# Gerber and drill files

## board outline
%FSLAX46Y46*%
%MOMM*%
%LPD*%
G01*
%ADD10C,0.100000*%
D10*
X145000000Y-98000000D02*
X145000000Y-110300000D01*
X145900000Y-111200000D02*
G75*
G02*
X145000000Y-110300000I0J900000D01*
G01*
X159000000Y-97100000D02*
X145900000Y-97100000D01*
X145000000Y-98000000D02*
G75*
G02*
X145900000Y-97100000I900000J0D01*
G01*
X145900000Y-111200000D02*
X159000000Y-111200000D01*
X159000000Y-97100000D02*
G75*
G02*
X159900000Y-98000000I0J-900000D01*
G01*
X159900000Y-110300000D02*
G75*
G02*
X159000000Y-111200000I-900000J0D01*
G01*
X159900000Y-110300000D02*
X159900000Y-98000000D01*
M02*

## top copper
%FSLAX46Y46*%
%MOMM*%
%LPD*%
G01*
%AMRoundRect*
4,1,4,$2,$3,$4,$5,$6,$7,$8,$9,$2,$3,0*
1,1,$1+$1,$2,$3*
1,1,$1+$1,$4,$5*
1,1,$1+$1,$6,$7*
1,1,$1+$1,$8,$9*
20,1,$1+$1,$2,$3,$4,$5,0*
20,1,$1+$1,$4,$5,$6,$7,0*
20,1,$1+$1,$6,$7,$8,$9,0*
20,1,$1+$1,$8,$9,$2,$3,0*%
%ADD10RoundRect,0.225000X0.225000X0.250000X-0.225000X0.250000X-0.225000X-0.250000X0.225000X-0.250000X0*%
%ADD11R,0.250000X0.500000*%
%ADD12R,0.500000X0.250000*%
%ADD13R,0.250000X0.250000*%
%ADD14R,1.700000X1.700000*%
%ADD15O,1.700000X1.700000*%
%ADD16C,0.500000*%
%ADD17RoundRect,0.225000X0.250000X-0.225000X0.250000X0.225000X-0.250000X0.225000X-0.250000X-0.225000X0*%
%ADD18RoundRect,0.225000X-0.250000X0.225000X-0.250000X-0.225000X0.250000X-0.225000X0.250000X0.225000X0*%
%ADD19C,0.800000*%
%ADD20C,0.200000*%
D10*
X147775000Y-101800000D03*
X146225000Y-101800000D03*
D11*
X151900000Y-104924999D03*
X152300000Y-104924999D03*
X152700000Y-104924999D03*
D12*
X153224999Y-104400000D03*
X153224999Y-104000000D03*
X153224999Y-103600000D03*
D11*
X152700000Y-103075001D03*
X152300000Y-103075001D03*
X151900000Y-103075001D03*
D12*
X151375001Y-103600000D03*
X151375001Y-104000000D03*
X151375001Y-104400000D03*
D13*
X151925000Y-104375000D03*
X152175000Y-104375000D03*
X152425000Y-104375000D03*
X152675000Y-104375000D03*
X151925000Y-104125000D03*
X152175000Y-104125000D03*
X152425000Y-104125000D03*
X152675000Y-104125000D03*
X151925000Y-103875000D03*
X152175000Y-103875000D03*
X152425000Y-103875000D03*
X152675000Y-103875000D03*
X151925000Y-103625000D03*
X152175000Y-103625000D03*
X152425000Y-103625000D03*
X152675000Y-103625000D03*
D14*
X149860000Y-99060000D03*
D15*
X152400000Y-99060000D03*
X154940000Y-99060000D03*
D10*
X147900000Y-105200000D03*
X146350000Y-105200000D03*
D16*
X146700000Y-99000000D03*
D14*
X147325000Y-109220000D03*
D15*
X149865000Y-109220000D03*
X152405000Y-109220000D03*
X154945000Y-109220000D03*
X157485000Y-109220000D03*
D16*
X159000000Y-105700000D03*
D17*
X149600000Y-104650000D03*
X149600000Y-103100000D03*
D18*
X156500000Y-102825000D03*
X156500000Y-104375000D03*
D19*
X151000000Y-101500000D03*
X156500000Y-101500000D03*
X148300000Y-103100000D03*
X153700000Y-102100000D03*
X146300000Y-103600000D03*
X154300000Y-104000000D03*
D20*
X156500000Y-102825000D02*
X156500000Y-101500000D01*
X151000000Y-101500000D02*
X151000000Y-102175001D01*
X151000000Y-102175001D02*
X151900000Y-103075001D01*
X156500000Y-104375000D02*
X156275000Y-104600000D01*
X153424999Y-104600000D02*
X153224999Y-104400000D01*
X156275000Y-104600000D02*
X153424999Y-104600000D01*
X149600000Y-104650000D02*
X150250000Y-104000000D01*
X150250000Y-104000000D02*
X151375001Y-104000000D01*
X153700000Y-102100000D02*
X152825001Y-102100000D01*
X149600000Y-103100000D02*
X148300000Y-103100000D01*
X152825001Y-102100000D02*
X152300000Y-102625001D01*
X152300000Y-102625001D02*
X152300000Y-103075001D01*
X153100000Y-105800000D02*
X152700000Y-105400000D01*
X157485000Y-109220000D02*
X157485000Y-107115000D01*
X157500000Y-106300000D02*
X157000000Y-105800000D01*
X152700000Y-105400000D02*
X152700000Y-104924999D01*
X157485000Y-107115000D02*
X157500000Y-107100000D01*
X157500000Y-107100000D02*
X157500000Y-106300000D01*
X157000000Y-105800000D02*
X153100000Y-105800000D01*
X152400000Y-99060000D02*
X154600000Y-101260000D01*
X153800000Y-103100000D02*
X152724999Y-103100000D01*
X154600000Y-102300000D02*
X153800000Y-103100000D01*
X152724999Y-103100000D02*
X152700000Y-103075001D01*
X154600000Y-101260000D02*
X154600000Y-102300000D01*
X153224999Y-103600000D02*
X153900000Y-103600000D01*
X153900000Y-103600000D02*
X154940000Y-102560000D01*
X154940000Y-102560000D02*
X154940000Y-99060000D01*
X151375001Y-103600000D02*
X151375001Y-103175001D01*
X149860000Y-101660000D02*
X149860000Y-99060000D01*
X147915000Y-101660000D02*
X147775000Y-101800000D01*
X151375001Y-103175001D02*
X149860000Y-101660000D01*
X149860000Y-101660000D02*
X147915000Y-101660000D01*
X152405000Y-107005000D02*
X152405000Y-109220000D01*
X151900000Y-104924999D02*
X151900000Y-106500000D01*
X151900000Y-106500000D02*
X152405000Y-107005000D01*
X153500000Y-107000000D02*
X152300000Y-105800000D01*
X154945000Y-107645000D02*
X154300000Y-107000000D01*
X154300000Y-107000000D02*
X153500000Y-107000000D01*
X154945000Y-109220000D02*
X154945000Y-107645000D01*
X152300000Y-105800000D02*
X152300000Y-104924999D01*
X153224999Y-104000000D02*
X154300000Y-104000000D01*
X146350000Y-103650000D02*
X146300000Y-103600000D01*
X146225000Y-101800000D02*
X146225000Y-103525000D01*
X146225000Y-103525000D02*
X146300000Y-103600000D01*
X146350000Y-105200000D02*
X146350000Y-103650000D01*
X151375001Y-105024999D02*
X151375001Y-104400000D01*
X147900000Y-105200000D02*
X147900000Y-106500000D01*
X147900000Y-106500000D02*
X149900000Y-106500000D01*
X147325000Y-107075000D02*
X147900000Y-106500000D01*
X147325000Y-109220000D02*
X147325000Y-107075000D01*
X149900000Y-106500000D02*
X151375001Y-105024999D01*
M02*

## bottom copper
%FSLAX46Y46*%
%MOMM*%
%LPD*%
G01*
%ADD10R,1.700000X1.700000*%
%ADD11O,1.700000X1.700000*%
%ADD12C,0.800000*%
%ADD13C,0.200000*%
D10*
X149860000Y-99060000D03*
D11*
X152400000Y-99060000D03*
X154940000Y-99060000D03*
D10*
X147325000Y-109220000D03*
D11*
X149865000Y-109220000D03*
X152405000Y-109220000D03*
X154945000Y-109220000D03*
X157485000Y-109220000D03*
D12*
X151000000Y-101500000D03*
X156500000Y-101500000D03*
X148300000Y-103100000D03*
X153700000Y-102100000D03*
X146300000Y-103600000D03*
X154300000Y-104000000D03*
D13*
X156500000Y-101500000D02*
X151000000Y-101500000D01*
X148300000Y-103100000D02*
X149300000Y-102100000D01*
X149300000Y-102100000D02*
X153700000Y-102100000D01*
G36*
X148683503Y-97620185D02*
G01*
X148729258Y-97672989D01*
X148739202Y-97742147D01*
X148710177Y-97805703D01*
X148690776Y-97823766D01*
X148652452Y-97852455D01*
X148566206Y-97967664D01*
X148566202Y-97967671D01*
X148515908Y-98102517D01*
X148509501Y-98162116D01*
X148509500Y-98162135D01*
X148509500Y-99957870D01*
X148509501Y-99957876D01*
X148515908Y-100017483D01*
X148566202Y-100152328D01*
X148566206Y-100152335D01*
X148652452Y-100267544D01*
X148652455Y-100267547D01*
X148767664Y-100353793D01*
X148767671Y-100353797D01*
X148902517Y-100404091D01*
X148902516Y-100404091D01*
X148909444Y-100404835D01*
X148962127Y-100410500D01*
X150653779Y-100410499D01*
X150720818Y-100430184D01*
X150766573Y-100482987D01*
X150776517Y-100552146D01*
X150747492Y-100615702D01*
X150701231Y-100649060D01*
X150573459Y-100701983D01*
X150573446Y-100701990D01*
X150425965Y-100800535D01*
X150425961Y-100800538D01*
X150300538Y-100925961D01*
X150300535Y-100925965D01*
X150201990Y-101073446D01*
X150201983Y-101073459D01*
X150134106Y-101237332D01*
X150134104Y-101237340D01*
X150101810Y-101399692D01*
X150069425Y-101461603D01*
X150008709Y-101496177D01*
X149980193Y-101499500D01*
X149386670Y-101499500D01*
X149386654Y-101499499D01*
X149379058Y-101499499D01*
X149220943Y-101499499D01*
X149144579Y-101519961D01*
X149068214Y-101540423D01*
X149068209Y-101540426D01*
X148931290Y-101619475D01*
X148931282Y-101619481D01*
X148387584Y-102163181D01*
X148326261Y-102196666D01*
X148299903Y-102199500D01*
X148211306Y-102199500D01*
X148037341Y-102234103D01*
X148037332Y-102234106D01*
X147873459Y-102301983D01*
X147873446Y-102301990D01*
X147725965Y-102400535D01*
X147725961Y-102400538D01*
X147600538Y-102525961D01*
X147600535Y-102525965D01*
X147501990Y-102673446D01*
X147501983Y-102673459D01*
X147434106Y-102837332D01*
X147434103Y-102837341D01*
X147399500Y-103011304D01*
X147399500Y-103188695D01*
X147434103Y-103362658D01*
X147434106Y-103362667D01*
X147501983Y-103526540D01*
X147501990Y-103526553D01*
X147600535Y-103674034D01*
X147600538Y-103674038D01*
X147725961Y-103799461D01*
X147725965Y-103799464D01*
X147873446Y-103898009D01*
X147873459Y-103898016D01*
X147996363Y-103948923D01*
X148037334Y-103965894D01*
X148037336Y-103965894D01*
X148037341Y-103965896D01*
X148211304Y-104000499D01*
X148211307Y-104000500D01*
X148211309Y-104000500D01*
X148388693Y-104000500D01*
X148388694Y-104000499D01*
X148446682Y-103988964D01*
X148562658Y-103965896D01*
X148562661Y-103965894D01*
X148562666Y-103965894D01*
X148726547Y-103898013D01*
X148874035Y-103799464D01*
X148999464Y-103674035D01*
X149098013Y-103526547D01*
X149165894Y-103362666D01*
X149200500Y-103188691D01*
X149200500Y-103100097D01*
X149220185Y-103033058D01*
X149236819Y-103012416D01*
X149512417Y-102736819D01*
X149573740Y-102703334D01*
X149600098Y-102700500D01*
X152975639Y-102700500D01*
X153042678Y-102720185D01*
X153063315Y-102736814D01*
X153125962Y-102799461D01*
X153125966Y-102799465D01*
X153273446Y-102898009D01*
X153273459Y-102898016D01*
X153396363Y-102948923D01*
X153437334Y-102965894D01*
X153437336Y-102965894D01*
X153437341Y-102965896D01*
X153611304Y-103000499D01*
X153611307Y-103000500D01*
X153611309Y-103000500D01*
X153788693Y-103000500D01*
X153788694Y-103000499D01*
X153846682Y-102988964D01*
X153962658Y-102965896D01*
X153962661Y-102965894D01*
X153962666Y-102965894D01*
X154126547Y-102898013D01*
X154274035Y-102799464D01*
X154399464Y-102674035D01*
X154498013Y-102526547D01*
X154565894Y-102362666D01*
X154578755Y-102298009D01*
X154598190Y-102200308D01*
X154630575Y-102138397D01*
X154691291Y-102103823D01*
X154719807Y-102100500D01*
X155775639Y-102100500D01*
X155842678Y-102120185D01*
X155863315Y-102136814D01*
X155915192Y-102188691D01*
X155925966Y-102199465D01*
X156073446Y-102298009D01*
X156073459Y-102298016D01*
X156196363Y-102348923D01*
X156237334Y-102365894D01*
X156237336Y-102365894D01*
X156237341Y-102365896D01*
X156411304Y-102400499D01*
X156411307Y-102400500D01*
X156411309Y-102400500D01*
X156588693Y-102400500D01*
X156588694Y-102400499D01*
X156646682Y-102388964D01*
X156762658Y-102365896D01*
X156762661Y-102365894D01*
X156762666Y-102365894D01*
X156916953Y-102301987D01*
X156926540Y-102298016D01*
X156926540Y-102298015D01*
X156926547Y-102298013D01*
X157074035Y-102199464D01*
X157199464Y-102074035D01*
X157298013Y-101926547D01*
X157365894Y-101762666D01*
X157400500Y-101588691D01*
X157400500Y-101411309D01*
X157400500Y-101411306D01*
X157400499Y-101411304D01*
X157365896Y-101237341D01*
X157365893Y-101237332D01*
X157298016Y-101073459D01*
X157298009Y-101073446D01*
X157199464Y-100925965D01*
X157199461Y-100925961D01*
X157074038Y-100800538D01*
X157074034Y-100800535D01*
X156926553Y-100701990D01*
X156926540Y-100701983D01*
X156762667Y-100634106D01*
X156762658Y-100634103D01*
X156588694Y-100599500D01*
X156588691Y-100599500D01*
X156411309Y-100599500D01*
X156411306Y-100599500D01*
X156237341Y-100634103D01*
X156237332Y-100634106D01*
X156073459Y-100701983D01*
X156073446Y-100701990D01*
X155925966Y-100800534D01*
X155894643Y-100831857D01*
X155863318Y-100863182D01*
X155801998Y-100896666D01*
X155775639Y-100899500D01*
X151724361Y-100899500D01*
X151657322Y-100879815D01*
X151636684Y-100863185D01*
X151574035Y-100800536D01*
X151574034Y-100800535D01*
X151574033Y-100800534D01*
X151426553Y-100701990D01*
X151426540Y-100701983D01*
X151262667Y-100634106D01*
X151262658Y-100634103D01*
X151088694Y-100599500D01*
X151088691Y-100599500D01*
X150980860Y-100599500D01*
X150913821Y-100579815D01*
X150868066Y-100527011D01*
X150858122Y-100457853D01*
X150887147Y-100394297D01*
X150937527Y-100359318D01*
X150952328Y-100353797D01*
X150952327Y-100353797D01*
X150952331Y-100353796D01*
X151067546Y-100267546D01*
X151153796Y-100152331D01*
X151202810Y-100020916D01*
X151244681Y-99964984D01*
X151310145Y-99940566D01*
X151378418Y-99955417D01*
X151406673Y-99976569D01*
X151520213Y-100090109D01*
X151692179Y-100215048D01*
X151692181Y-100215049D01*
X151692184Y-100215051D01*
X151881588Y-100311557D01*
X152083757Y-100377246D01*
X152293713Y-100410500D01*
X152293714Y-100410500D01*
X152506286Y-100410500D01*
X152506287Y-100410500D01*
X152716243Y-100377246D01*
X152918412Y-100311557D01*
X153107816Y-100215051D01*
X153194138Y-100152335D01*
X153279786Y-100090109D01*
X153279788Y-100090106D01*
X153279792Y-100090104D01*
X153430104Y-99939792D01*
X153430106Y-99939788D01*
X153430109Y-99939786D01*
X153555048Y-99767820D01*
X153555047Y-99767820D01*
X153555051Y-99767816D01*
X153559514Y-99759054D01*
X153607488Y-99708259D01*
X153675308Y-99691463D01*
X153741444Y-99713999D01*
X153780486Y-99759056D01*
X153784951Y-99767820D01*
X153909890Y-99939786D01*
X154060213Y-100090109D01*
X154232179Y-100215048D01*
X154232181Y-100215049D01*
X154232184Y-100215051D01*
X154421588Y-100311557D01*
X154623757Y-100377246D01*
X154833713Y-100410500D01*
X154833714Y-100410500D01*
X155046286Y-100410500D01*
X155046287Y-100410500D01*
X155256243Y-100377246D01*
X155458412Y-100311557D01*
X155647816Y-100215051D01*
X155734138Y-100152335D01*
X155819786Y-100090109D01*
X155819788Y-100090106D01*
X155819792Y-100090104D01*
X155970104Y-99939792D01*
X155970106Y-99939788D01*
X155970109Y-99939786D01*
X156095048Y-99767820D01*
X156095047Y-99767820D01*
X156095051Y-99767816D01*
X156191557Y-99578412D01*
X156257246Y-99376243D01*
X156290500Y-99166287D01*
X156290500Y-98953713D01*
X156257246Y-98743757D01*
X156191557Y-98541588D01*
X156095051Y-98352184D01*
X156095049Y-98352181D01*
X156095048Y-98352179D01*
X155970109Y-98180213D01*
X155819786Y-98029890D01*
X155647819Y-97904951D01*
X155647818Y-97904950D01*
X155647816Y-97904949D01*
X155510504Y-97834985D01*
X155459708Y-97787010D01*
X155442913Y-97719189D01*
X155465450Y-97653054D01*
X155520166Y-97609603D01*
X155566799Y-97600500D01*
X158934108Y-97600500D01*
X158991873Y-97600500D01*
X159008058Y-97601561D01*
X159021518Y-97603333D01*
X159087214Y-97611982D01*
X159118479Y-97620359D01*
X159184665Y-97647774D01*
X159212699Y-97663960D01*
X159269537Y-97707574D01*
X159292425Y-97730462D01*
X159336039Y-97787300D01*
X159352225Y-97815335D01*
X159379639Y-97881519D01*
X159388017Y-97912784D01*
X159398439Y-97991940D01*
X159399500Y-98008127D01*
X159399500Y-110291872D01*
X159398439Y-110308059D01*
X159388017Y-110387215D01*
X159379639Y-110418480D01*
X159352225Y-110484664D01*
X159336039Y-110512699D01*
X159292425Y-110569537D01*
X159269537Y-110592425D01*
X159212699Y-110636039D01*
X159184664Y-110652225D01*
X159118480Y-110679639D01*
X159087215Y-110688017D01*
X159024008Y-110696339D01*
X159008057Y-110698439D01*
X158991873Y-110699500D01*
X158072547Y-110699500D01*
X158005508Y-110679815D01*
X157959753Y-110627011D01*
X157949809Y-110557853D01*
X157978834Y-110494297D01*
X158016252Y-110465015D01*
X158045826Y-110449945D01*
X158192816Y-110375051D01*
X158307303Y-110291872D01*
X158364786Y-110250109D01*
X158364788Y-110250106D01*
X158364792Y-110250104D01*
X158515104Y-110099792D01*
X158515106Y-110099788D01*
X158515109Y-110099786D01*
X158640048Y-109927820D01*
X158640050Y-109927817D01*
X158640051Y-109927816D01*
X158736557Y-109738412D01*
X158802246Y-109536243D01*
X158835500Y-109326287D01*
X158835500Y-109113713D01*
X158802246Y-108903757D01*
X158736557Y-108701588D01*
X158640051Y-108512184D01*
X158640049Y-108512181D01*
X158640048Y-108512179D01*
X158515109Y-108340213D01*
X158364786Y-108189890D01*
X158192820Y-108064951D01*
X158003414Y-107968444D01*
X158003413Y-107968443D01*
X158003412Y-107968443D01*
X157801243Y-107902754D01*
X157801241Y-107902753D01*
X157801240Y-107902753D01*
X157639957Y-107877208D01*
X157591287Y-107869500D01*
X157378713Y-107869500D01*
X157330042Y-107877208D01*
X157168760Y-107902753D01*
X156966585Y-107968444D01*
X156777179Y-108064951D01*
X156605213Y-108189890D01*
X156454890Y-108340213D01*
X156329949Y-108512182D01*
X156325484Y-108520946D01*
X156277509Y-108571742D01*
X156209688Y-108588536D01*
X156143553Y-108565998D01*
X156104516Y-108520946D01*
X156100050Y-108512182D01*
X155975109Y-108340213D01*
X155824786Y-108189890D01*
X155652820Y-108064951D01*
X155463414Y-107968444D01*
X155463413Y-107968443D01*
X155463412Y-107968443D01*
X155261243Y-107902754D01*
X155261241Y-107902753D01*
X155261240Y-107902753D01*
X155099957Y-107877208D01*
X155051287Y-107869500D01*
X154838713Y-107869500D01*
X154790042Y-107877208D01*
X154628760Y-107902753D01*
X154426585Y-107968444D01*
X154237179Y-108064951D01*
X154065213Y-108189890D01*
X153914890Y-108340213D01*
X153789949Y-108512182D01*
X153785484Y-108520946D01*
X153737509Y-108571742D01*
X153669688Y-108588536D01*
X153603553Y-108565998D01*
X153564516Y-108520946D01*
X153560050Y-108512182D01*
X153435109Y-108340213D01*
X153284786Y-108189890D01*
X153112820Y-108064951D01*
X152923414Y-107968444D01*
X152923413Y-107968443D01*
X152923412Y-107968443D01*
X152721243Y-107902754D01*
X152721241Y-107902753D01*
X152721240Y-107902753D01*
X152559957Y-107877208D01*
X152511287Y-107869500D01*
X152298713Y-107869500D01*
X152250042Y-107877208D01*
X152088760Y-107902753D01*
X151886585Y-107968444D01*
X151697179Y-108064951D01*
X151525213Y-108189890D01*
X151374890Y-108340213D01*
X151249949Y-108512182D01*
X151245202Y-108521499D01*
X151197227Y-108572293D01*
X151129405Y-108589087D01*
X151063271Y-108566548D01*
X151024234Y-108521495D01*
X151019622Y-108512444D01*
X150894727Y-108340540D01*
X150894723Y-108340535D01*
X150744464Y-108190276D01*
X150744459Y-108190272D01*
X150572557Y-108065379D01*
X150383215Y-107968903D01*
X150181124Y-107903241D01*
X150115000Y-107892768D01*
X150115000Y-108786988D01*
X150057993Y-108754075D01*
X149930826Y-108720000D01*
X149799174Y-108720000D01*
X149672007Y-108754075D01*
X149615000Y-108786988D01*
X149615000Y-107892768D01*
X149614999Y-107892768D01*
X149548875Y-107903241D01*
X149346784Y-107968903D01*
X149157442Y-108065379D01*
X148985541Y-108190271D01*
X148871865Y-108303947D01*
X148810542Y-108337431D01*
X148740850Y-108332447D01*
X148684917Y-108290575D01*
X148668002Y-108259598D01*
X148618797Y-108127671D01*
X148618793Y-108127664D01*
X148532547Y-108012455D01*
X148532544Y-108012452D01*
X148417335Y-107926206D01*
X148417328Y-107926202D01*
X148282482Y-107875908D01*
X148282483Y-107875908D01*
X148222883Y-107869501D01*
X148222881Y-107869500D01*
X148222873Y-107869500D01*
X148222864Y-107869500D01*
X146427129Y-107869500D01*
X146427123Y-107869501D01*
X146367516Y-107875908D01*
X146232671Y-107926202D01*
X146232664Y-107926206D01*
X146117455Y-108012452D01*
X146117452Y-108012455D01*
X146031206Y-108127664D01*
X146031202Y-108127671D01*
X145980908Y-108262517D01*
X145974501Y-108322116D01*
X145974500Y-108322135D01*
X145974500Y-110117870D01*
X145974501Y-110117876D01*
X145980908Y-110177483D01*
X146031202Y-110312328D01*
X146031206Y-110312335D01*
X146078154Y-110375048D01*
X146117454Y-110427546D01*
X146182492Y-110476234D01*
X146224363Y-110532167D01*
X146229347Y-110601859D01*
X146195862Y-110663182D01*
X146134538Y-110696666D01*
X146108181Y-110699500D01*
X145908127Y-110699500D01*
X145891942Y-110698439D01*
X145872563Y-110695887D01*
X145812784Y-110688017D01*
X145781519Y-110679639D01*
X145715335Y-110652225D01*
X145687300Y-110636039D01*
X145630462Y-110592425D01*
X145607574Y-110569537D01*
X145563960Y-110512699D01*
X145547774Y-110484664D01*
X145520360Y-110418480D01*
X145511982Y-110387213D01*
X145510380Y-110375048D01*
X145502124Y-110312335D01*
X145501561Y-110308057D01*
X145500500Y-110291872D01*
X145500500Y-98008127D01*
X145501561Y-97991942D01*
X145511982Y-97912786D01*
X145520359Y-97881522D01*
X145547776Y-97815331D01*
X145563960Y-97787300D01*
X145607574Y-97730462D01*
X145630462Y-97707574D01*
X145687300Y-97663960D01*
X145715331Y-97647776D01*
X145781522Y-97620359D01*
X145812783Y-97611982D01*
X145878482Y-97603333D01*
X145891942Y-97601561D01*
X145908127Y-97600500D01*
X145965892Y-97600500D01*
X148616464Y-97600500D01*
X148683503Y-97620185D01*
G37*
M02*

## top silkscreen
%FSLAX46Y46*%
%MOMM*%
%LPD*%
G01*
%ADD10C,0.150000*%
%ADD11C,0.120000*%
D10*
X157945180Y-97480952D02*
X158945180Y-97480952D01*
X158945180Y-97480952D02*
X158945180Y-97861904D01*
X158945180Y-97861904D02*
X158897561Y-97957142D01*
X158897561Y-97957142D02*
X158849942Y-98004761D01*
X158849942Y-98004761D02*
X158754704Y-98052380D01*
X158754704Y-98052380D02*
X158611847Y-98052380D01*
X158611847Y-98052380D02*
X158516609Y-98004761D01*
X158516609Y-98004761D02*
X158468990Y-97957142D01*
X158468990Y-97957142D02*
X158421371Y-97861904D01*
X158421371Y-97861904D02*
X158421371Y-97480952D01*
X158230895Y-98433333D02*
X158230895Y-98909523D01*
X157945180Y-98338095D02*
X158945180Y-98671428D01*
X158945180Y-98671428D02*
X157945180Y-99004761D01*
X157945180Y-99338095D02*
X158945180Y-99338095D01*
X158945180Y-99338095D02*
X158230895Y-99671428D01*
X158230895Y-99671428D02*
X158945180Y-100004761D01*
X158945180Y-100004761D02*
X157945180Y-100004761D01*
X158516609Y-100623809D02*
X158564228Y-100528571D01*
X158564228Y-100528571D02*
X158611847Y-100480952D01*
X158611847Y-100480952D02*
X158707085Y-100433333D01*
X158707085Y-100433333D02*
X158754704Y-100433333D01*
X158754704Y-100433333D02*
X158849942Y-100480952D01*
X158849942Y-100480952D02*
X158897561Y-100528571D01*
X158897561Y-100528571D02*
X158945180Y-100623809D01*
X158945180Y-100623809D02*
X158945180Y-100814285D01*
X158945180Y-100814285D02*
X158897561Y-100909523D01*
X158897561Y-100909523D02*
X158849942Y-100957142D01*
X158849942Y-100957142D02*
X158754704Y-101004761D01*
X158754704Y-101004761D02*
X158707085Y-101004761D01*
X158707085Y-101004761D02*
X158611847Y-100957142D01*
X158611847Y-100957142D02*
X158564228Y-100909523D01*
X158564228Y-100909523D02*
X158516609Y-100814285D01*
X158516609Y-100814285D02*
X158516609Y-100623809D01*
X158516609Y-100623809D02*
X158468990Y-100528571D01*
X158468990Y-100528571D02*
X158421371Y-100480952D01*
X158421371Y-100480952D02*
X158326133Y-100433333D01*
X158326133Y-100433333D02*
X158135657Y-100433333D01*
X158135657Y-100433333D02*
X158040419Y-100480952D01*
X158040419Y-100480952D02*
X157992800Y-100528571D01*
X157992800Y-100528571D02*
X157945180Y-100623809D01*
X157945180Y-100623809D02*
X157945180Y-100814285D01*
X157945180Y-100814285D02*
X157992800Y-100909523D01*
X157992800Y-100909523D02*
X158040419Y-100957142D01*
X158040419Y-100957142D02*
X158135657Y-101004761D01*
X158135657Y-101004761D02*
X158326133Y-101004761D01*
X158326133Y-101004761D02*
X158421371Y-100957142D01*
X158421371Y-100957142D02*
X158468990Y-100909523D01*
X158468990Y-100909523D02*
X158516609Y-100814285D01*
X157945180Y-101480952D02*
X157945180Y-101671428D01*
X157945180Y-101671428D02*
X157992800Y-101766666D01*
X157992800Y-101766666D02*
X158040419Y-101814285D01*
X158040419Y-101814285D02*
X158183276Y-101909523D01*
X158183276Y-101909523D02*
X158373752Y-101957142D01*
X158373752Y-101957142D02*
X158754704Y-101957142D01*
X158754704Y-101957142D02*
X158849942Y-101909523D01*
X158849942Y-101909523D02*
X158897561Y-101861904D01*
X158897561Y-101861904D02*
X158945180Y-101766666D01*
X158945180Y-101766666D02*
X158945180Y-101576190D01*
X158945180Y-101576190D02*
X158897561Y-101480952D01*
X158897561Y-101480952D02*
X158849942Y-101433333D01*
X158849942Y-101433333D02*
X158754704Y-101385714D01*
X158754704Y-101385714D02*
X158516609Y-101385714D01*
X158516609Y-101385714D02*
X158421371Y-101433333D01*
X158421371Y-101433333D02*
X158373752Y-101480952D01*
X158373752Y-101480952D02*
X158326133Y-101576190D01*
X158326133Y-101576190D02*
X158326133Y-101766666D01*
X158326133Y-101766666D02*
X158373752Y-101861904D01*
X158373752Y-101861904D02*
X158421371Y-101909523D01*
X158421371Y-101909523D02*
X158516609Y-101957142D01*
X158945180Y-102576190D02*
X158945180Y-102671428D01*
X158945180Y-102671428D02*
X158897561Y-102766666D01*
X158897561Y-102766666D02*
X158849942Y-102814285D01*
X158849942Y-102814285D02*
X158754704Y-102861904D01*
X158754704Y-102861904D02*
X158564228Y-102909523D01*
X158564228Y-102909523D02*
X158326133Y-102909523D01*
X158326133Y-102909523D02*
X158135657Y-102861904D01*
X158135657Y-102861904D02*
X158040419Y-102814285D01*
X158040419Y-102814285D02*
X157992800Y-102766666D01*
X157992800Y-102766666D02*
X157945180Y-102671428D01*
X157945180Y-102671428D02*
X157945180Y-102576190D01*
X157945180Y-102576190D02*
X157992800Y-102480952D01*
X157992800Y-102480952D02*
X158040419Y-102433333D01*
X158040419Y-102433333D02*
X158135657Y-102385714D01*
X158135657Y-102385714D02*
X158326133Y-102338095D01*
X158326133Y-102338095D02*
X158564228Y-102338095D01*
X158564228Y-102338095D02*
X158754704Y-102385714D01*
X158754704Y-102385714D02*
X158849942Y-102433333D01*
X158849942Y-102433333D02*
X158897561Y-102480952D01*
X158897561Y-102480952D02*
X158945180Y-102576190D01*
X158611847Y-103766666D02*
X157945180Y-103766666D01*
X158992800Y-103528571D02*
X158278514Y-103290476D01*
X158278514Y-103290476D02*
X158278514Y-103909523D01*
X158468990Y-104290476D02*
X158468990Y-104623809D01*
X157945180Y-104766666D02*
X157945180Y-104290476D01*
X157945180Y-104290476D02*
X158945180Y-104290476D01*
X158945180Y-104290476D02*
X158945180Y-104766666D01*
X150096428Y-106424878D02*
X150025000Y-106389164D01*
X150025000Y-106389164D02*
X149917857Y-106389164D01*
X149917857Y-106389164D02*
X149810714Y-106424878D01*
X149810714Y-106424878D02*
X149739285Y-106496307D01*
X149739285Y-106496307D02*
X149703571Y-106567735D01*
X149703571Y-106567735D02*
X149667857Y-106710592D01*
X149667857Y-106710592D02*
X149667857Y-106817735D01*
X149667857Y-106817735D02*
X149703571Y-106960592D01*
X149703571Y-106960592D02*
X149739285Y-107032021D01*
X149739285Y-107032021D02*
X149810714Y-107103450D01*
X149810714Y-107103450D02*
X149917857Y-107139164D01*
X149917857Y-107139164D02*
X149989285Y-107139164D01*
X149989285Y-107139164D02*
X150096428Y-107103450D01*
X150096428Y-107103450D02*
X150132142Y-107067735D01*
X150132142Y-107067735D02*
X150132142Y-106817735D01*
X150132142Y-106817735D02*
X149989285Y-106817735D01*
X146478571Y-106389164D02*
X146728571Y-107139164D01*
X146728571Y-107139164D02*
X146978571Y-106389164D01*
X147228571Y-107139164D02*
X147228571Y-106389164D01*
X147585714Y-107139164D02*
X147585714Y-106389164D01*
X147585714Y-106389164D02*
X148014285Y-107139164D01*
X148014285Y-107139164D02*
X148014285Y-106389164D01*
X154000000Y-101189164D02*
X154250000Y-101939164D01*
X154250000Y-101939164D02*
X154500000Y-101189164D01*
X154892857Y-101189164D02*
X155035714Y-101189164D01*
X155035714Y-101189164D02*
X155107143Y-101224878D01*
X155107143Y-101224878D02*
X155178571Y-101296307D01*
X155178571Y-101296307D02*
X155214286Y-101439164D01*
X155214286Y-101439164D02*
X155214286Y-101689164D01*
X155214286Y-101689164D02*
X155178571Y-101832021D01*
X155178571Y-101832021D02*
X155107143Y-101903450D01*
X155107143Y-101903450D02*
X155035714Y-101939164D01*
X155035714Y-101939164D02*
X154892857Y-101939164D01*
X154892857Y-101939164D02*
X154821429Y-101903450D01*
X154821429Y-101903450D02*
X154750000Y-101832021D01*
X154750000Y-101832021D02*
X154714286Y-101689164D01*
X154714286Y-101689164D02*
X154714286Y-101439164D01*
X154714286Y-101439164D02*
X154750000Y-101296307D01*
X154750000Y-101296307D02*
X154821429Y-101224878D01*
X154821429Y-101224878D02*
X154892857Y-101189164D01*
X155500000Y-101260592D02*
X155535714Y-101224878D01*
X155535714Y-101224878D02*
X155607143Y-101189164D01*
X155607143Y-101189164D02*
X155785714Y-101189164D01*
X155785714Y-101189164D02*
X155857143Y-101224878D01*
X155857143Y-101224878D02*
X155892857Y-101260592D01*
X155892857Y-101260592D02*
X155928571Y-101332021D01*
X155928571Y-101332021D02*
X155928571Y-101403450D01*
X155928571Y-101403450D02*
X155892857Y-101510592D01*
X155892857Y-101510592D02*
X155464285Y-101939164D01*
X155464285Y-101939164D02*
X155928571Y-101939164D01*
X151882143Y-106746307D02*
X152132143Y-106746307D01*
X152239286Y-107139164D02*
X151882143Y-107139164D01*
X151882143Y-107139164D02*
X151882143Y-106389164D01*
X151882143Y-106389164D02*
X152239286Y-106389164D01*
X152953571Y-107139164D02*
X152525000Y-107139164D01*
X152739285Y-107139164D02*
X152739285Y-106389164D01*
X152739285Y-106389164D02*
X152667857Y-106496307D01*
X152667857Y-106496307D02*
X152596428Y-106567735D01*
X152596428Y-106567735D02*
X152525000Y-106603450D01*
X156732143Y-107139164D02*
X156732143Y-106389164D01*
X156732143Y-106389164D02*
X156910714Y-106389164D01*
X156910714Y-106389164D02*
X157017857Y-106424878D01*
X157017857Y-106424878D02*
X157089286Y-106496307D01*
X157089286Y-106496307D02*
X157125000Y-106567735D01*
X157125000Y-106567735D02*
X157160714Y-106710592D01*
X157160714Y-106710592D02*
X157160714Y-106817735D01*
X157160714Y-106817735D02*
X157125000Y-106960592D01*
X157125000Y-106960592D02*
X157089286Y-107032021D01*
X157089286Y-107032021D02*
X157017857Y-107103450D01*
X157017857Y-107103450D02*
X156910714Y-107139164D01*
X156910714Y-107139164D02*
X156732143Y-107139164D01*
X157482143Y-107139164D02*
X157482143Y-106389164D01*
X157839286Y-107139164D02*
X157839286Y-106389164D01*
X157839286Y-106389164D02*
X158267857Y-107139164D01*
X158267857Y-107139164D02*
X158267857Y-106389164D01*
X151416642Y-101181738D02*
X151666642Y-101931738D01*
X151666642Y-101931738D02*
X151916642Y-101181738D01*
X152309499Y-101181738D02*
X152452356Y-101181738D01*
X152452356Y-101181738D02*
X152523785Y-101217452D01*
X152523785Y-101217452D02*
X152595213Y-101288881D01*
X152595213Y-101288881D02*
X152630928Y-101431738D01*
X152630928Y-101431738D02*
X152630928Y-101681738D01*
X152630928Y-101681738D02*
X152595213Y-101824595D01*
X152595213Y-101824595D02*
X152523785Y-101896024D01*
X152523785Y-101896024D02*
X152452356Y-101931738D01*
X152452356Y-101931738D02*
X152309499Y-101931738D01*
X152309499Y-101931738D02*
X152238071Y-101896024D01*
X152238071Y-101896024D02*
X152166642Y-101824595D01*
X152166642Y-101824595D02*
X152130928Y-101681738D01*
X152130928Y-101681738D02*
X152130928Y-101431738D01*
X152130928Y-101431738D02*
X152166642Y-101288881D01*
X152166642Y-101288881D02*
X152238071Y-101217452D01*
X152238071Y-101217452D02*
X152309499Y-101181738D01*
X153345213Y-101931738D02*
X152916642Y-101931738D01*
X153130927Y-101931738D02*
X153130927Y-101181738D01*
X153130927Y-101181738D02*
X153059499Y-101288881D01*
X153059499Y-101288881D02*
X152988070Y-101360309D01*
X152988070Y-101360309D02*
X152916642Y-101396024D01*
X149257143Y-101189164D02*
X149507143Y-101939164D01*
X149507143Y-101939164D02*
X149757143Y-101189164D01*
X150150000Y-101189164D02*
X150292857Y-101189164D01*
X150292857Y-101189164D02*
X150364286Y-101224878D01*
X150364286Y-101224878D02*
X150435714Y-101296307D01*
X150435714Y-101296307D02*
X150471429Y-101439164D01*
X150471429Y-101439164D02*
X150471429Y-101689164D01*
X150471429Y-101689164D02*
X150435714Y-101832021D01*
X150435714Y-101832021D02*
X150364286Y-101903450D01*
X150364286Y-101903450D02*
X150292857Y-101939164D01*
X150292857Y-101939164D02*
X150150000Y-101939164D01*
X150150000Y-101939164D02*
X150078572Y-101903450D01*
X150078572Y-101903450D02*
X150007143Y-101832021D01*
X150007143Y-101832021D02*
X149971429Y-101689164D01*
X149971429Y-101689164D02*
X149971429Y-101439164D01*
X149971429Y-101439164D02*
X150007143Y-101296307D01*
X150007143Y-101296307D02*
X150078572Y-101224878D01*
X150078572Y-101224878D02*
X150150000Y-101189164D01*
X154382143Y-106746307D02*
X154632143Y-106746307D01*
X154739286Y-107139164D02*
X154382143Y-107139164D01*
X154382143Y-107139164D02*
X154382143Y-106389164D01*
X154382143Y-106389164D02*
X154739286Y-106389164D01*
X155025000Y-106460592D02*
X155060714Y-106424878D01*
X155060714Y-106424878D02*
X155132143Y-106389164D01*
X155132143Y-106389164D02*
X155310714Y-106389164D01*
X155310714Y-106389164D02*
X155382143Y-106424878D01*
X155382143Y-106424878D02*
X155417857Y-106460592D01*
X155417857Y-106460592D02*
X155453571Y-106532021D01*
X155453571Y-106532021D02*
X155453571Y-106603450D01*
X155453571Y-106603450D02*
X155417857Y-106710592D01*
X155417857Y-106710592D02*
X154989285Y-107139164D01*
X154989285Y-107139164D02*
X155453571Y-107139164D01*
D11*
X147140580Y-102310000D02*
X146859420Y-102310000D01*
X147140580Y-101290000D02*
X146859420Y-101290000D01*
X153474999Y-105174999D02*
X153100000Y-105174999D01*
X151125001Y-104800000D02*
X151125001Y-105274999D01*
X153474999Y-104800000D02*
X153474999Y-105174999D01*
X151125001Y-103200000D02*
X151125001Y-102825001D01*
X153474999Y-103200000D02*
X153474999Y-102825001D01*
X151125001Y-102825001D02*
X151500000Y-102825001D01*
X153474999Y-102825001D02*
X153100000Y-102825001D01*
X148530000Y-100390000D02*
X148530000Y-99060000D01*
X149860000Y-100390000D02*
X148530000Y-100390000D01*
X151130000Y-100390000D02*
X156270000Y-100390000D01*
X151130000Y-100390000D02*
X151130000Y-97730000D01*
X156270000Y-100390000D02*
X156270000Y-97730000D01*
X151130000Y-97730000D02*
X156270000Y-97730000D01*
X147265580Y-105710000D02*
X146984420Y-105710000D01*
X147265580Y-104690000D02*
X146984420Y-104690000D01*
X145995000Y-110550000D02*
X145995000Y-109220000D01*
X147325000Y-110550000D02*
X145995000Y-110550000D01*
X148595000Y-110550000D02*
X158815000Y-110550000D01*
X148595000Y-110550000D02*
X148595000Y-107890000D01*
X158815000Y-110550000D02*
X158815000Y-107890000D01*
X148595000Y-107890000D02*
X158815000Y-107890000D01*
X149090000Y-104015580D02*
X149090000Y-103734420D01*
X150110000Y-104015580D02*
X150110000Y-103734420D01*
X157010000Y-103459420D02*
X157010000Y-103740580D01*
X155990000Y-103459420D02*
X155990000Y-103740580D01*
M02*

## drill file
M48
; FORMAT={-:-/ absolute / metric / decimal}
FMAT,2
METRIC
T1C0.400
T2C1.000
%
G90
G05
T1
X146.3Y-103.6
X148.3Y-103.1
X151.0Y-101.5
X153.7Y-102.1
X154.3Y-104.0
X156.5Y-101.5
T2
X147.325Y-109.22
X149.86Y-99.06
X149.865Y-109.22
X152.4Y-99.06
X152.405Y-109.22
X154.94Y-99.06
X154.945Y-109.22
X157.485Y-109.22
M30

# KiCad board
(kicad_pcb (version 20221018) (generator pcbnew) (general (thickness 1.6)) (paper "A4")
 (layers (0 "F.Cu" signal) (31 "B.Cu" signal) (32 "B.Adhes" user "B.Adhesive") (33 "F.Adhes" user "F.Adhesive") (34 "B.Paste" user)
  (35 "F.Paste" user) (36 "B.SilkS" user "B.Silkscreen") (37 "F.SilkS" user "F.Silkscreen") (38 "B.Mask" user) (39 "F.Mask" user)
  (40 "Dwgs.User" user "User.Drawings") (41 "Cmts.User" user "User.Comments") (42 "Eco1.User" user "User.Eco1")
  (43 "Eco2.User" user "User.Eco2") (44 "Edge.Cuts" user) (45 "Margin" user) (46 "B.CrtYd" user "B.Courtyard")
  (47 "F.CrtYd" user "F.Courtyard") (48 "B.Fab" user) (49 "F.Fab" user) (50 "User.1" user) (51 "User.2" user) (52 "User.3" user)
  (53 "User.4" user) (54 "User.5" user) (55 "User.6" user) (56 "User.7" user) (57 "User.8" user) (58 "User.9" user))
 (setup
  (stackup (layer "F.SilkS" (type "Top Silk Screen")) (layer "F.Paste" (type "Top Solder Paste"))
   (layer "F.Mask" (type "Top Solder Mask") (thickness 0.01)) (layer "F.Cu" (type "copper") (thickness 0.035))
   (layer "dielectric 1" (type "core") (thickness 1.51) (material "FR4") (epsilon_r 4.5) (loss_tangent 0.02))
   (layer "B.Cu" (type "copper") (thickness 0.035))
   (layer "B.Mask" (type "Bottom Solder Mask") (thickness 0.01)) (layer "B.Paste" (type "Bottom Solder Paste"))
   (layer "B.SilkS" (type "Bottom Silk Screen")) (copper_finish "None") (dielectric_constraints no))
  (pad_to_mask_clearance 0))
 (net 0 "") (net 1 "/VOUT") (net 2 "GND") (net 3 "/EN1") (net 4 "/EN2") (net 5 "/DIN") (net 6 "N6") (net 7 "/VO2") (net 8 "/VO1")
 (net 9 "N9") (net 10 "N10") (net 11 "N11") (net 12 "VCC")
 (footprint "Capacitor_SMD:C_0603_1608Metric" (layer "F.Cu") (at 147 101.8 180)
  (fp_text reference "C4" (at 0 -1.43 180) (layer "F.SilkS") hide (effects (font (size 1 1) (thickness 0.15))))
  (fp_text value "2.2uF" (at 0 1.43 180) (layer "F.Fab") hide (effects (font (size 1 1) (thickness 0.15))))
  (fp_line (start -0.14058 -0.51) (end 0.14058 -0.51) (stroke (width 0.12) (type solid)) (layer "F.SilkS"))
  (fp_line (start -0.14058 0.51) (end 0.14058 0.51) (stroke (width 0.12) (type solid)) (layer "F.SilkS"))
  (pad "1" smd roundrect (at -0.775 0 180) (size 0.9 0.95) (layers "F.Cu" "F.Paste" "F.Mask") (roundrect_rratio 0.25) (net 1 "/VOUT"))
  (pad "2" smd roundrect (at 0.775 0 180) (size 0.9 0.95) (layers "F.Cu" "F.Paste" "F.Mask") (roundrect_rratio 0.25) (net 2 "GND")))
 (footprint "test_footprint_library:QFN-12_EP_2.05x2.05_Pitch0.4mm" (layer "F.Cu") (at 152.3 104 90) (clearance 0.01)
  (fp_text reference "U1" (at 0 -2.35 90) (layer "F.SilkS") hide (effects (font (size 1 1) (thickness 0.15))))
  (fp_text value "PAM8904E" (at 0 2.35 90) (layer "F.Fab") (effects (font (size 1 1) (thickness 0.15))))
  (fp_line (start -1.174999 1.174999) (end -1.174999 0.8) (stroke (width 0.12) (type default)) (layer "F.SilkS"))
  (fp_line (start -0.8 -1.174999) (end -1.274999 -1.174999) (stroke (width 0.12) (type default)) (layer "F.SilkS"))
  (fp_line (start -0.8 1.174999) (end -1.174999 1.174999) (stroke (width 0.12) (type default)) (layer "F.SilkS"))
  (fp_line (start 0.8 -1.174999) (end 1.174999 -1.174999) (stroke (width 0.12) (type default)) (layer "F.SilkS"))
  (fp_line (start 0.8 1.174999) (end 1.174999 1.174999) (stroke (width 0.12) (type default)) (layer "F.SilkS"))
  (fp_line (start 1.174999 -1.174999) (end 1.174999 -0.8) (stroke (width 0.12) (type default)) (layer "F.SilkS"))
  (fp_line (start 1.174999 1.174999) (end 1.174999 0.8) (stroke (width 0.12) (type default)) (layer "F.SilkS"))
  (pad "1" smd rect (at -0.924999 -0.4 180) (size 0.25 0.5) (layers "F.Cu" "F.Paste" "F.Mask") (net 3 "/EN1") (thermal_bridge_angle 45))
  (pad "2" smd rect (at -0.924999 0 180) (size 0.25 0.5) (layers "F.Cu" "F.Paste" "F.Mask") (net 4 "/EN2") (thermal_bridge_angle 45))
  (pad "3" smd rect (at -0.924999 0.4 180) (size 0.25 0.5) (layers "F.Cu" "F.Paste" "F.Mask") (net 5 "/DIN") (thermal_bridge_angle 45))
  (pad "4" smd rect (at -0.4 0.924999 90) (size 0.25 0.5) (layers "F.Cu" "F.Paste" "F.Mask") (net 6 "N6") (thermal_bridge_angle 45))
  (pad "5" smd rect (at 0 0.924999 90) (size 0.25 0.5) (layers "F.Cu" "F.Paste" "F.Mask") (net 2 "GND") (thermal_bridge_angle 45))
  (pad "6" smd rect (at 0.4 0.924999 90) (size 0.25 0.5) (layers "F.Cu" "F.Paste" "F.Mask") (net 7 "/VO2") (thermal_bridge_angle 45))
  (pad "7" smd rect (at 0.924999 0.4 180) (size 0.25 0.5) (layers "F.Cu" "F.Paste" "F.Mask") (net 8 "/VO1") (thermal_bridge_angle 45))
  (pad "8" smd rect (at 0.924999 0 180) (size 0.25 0.5) (layers "F.Cu" "F.Paste" "F.Mask") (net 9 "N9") (thermal_bridge_angle 45))
  (pad "9" smd rect (at 0.924999 -0.4 180) (size 0.25 0.5) (layers "F.Cu" "F.Paste" "F.Mask") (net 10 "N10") (thermal_bridge_angle 45))
  (pad "10" smd rect (at 0.4 -0.924999 90) (size 0.25 0.5) (layers "F.Cu" "F.Paste" "F.Mask") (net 1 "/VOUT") (thermal_bridge_angle 45))
  (pad "11" smd rect (at 0 -0.924999 90) (size 0.25 0.5) (layers "F.Cu" "F.Paste" "F.Mask") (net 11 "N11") (thermal_bridge_angle 45))
  (pad "12" smd rect (at -0.4 -0.924999 90) (size 0.25 0.5) (layers "F.Cu" "F.Paste" "F.Mask") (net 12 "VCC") (thermal_bridge_angle 45))
  (pad "13" smd rect (at -0.375 -0.375 90) (size 0.25 0.25) (layers "F.Cu" "F.Paste" "F.Mask") (solder_paste_margin -0.75)
   (thermal_bridge_angle 45))
  (pad "13" smd rect (at -0.375 -0.125 90) (size 0.25 0.25) (layers "F.Cu" "F.Paste" "F.Mask") (solder_paste_margin -0.75)
   (thermal_bridge_angle 45))
  (pad "13" smd rect (at -0.375 0.125 90) (size 0.25 0.25) (layers "F.Cu" "F.Paste" "F.Mask") (solder_paste_margin -0.75)
   (thermal_bridge_angle 45))
  (pad "13" smd rect (at -0.375 0.375 90) (size 0.25 0.25) (layers "F.Cu" "F.Paste" "F.Mask") (solder_paste_margin -0.75)
   (thermal_bridge_angle 45))
  (pad "13" smd rect (at -0.125 -0.375 90) (size 0.25 0.25) (layers "F.Cu" "F.Paste" "F.Mask") (solder_paste_margin -0.75)
   (thermal_bridge_angle 45))
  (pad "13" smd rect (at -0.125 -0.125 90) (size 0.25 0.25) (layers "F.Cu" "F.Paste" "F.Mask") (solder_paste_margin -0.75)
   (thermal_bridge_angle 45))
  (pad "13" smd rect (at -0.125 0.125 90) (size 0.25 0.25) (layers "F.Cu" "F.Paste" "F.Mask") (solder_paste_margin -0.75)
   (thermal_bridge_angle 45))
  (pad "13" smd rect (at -0.125 0.375 90) (size 0.25 0.25) (layers "F.Cu" "F.Paste" "F.Mask") (solder_paste_margin -0.75)
   (thermal_bridge_angle 45))
  (pad "13" smd rect (at 0.125 -0.375 90) (size 0.25 0.25) (layers "F.Cu" "F.Paste" "F.Mask") (solder_paste_margin -0.75)
   (thermal_bridge_angle 45))
  (pad "13" smd rect (at 0.125 -0.125 90) (size 0.25 0.25) (layers "F.Cu" "F.Paste" "F.Mask") (solder_paste_margin -0.75)
   (thermal_bridge_angle 45))
  (pad "13" smd rect (at 0.125 0.125 90) (size 0.25 0.25) (layers "F.Cu" "F.Paste" "F.Mask") (solder_paste_margin -0.75)
   (thermal_bridge_angle 45))
  (pad "13" smd rect (at 0.125 0.375 90) (size 0.25 0.25) (layers "F.Cu" "F.Paste" "F.Mask") (solder_paste_margin -0.75)
   (thermal_bridge_angle 45))
  (pad "13" smd rect (at 0.375 -0.375 90) (size 0.25 0.25) (layers "F.Cu" "F.Paste" "F.Mask") (solder_paste_margin -0.75)
   (thermal_bridge_angle 45))
  (pad "13" smd rect (at 0.375 -0.125 90) (size 0.25 0.25) (layers "F.Cu" "F.Paste" "F.Mask") (solder_paste_margin -0.75)
   (thermal_bridge_angle 45))
  (pad "13" smd rect (at 0.375 0.125 90) (size 0.25 0.25) (layers "F.Cu" "F.Paste" "F.Mask") (solder_paste_margin -0.75)
   (thermal_bridge_angle 45))
  (pad "13" smd rect (at 0.375 0.375 90) (size 0.25 0.25) (layers "F.Cu" "F.Paste" "F.Mask") (solder_paste_margin -0.75)
   (thermal_bridge_angle 45)))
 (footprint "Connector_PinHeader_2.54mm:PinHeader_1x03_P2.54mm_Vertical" (layer "F.Cu") (at 149.86 99.06 90)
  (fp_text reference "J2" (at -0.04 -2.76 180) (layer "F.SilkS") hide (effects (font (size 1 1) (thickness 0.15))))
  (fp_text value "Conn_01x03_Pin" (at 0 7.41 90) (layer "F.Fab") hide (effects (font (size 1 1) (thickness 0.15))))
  (fp_line (start -1.33 -1.33) (end 0 -1.33) (stroke (width 0.12) (type solid)) (layer "F.SilkS"))
  (fp_line (start -1.33 0) (end -1.33 -1.33) (stroke (width 0.12) (type solid)) (layer "F.SilkS"))
  (fp_line (start -1.33 1.27) (end -1.33 6.41) (stroke (width 0.12) (type solid)) (layer "F.SilkS"))
  (fp_line (start -1.33 1.27) (end 1.33 1.27) (stroke (width 0.12) (type solid)) (layer "F.SilkS"))
  (fp_line (start -1.33 6.41) (end 1.33 6.41) (stroke (width 0.12) (type solid)) (layer "F.SilkS"))
  (fp_line (start 1.33 1.27) (end 1.33 6.41) (stroke (width 0.12) (type solid)) (layer "F.SilkS"))
  (pad "1" thru_hole rect (at 0 0 90) (size 1.7 1.7) (drill 1) (layers "*.Cu" "*.Mask") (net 1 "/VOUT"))
  (pad "2" thru_hole oval (at 0 2.54 90) (size 1.7 1.7) (drill 1) (layers "*.Cu" "*.Mask") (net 8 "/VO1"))
  (pad "3" thru_hole oval (at 0 5.08 90) (size 1.7 1.7) (drill 1) (layers "*.Cu" "*.Mask") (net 7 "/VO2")))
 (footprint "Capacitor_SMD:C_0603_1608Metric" (layer "F.Cu") (at 147.125 105.2 180)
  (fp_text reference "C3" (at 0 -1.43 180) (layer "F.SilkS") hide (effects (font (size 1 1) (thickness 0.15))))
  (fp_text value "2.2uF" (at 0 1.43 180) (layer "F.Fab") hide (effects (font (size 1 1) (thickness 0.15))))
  (fp_line (start -0.14058 -0.51) (end 0.14058 -0.51) (stroke (width 0.12) (type solid)) (layer "F.SilkS"))
  (fp_line (start -0.14058 0.51) (end 0.14058 0.51) (stroke (width 0.12) (type solid)) (layer "F.SilkS"))
  (pad "1" smd roundrect (at -0.775 0 180) (size 0.9 0.95) (layers "F.Cu" "F.Paste" "F.Mask") (roundrect_rratio 0.25) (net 12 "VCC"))
  (pad "2" smd roundrect (at 0.775 0 180) (size 0.9 0.95) (layers "F.Cu" "F.Paste" "F.Mask") (roundrect_rratio 0.25) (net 2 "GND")))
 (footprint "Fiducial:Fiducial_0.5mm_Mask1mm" (layer "F.Cu") (at 146.7 99)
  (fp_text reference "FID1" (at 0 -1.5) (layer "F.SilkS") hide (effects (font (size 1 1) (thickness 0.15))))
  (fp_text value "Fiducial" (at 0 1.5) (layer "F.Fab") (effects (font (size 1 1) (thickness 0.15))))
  (pad "" smd circle (at 0 0) (size 0.5 0.5) (layers "F.Cu" "F.Mask") (solder_mask_margin 0.25) (clearance 0.25)))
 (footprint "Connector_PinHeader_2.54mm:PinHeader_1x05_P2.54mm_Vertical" (layer "F.Cu") (at 147.325 109.22 90)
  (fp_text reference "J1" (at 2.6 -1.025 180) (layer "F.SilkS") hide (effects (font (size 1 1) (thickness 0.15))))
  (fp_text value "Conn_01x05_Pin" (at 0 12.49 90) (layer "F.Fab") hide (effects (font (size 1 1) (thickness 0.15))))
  (fp_line (start -1.33 -1.33) (end 0 -1.33) (stroke (width 0.12) (type solid)) (layer "F.SilkS"))
  (fp_line (start -1.33 0) (end -1.33 -1.33) (stroke (width 0.12) (type solid)) (layer "F.SilkS"))
  (fp_line (start -1.33 1.27) (end -1.33 11.49) (stroke (width 0.12) (type solid)) (layer "F.SilkS"))
  (fp_line (start -1.33 1.27) (end 1.33 1.27) (stroke (width 0.12) (type solid)) (layer "F.SilkS"))
  (fp_line (start -1.33 11.49) (end 1.33 11.49) (stroke (width 0.12) (type solid)) (layer "F.SilkS"))
  (fp_line (start 1.33 1.27) (end 1.33 11.49) (stroke (width 0.12) (type solid)) (layer "F.SilkS"))
  (pad "1" thru_hole rect (at 0 0 90) (size 1.7 1.7) (drill 1) (layers "*.Cu" "*.Mask") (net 12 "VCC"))
  (pad "2" thru_hole oval (at 0 2.54 90) (size 1.7 1.7) (drill 1) (layers "*.Cu" "*.Mask") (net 2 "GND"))
  (pad "3" thru_hole oval (at 0 5.08 90) (size 1.7 1.7) (drill 1) (layers "*.Cu" "*.Mask") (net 3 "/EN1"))
  (pad "4" thru_hole oval (at 0 7.62 90) (size 1.7 1.7) (drill 1) (layers "*.Cu" "*.Mask") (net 4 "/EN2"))
  (pad "5" thru_hole oval (at 0 10.16 90) (size 1.7 1.7) (drill 1) (layers "*.Cu" "*.Mask") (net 5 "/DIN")))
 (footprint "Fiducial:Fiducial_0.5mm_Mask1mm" (layer "F.Cu") (at 159 105.7)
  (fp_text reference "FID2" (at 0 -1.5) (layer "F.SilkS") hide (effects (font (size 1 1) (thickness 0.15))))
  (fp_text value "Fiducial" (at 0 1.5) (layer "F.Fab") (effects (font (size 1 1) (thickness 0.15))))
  (pad "" smd circle (at 0 0) (size 0.5 0.5) (layers "F.Cu" "F.Mask") (solder_mask_margin 0.25) (clearance 0.25)))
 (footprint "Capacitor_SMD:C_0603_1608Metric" (layer "F.Cu") (at 149.6 103.875 90)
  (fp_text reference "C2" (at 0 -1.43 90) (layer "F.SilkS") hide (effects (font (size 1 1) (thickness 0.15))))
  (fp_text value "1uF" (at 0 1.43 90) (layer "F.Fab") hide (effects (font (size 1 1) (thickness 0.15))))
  (fp_line (start -0.14058 -0.51) (end 0.14058 -0.51) (stroke (width 0.12) (type solid)) (layer "F.SilkS"))
  (fp_line (start -0.14058 0.51) (end 0.14058 0.51) (stroke (width 0.12) (type solid)) (layer "F.SilkS"))
  (pad "1" smd roundrect (at -0.775 0 90) (size 0.9 0.95) (layers "F.Cu" "F.Paste" "F.Mask") (roundrect_rratio 0.25) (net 11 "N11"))
  (pad "2" smd roundrect (at 0.775 0 90) (size 0.9 0.95) (layers "F.Cu" "F.Paste" "F.Mask") (roundrect_rratio 0.25) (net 9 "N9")))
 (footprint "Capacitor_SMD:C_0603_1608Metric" (layer "F.Cu") (at 156.5 103.6 -90)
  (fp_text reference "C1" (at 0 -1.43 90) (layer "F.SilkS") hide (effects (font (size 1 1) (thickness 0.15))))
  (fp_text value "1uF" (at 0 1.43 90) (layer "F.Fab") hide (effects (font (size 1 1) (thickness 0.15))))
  (fp_line (start -0.14058 -0.51) (end 0.14058 -0.51) (stroke (width 0.12) (type solid)) (layer "F.SilkS"))
  (fp_line (start -0.14058 0.51) (end 0.14058 0.51) (stroke (width 0.12) (type solid)) (layer "F.SilkS"))
  (pad "1" smd roundrect (at -0.775 0 270) (size 0.9 0.95) (layers "F.Cu" "F.Paste" "F.Mask") (roundrect_rratio 0.25) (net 10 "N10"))
  (pad "2" smd roundrect (at 0.775 0 270) (size 0.9 0.95) (layers "F.Cu" "F.Paste" "F.Mask") (roundrect_rratio 0.25) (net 6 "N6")))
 (gr_line (start 145 98) (end 145 110.3) (stroke (width 0.1) (type default)) (layer "Edge.Cuts"))
 (gr_arc (start 145.9 111.2) (mid 145.263604 110.936396) (end 145 110.3) (stroke (width 0.1) (type default)) (layer "Edge.Cuts"))
 (gr_line (start 159 97.1) (end 145.9 97.1) (stroke (width 0.1) (type default)) (layer "Edge.Cuts"))
 (gr_arc (start 145 98) (mid 145.263604 97.363604) (end 145.9 97.1) (stroke (width 0.1) (type default)) (layer "Edge.Cuts"))
 (gr_line (start 145.9 111.2) (end 159 111.2) (stroke (width 0.1) (type default)) (layer "Edge.Cuts"))
 (gr_arc (start 159 97.1) (mid 159.636396 97.363604) (end 159.9 98) (stroke (width 0.1) (type default)) (layer "Edge.Cuts"))
 (gr_arc (start 159.9 110.3) (mid 159.636396 110.936396) (end 159 111.2) (stroke (width 0.1) (type default)) (layer "Edge.Cuts"))
 (gr_line (start 159.9 110.3) (end 159.9 98) (stroke (width 0.1) (type default)) (layer "Edge.Cuts"))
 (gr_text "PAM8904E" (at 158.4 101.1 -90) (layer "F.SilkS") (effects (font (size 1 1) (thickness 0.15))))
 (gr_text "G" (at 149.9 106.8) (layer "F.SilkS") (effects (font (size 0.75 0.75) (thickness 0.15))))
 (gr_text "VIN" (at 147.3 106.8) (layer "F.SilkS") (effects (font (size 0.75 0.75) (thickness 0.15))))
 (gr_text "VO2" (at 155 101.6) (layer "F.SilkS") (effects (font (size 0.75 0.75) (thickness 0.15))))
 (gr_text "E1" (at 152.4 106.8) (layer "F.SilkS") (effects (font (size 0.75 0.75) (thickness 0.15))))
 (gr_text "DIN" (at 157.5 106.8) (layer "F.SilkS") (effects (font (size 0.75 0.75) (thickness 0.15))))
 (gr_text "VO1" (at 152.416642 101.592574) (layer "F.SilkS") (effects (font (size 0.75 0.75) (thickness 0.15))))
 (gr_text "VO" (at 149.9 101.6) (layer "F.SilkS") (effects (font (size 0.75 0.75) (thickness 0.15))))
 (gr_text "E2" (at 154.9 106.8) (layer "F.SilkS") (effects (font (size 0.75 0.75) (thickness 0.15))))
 (segment (start 156.5 102.825) (end 156.5 101.5) (width 0.2) (layer "F.Cu") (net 10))
 (segment (start 151 101.5) (end 151 102.175001) (width 0.2) (layer "F.Cu") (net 10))
 (segment (start 151 102.175001) (end 151.9 103.075001) (width 0.2) (layer "F.Cu") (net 10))
 (via (at 151 101.5) (size 0.8) (drill 0.4) (layers "F.Cu" "B.Cu") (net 10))
 (via (at 156.5 101.5) (size 0.8) (drill 0.4) (layers "F.Cu" "B.Cu") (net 10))
 (segment (start 156.5 101.5) (end 151 101.5) (width 0.2) (layer "B.Cu") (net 10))
 (segment (start 156.5 104.375) (end 156.275 104.6) (width 0.2) (layer "F.Cu") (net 6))
 (segment (start 153.424999 104.6) (end 153.224999 104.4) (width 0.2) (layer "F.Cu") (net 6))
 (segment (start 156.275 104.6) (end 153.424999 104.6) (width 0.2) (layer "F.Cu") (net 6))
 (segment (start 149.6 104.65) (end 150.25 104) (width 0.2) (layer "F.Cu") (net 11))
 (segment (start 150.25 104) (end 151.375001 104) (width 0.2) (layer "F.Cu") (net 11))
 (segment (start 153.7 102.1) (end 152.825001 102.1) (width 0.2) (layer "F.Cu") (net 9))
 (segment (start 149.6 103.1) (end 148.3 103.1) (width 0.2) (layer "F.Cu") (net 9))
 (segment (start 152.825001 102.1) (end 152.3 102.625001) (width 0.2) (layer "F.Cu") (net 9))
 (segment (start 152.3 102.625001) (end 152.3 103.075001) (width 0.2) (layer "F.Cu") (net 9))
 (via (at 148.3 103.1) (size 0.8) (drill 0.4) (layers "F.Cu" "B.Cu") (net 9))
 (via (at 153.7 102.1) (size 0.8) (drill 0.4) (layers "F.Cu" "B.Cu") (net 9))
 (segment (start 148.3 103.1) (end 149.3 102.1) (width 0.2) (layer "B.Cu") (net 9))
 (segment (start 149.3 102.1) (end 153.7 102.1) (width 0.2) (layer "B.Cu") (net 9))
 (segment (start 153.1 105.8) (end 152.7 105.4) (width 0.2) (layer "F.Cu") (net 5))
 (segment (start 157.485 109.22) (end 157.485 107.115) (width 0.2) (layer "F.Cu") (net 5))
 (segment (start 157.5 106.3) (end 157 105.8) (width 0.2) (layer "F.Cu") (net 5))
 (segment (start 152.7 105.4) (end 152.7 104.924999) (width 0.2) (layer "F.Cu") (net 5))
 (segment (start 157.485 107.115) (end 157.5 107.1) (width 0.2) (layer "F.Cu") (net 5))
 (segment (start 157.5 107.1) (end 157.5 106.3) (width 0.2) (layer "F.Cu") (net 5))
 (segment (start 157 105.8) (end 153.1 105.8) (width 0.2) (layer "F.Cu") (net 5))
 (segment (start 152.4 99.06) (end 154.6 101.26) (width 0.2) (layer "F.Cu") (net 8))
 (segment (start 153.8 103.1) (end 152.724999 103.1) (width 0.2) (layer "F.Cu") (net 8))
 (segment (start 154.6 102.3) (end 153.8 103.1) (width 0.2) (layer "F.Cu") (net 8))
 (segment (start 152.724999 103.1) (end 152.7 103.075001) (width 0.2) (layer "F.Cu") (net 8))
 (segment (start 154.6 101.26) (end 154.6 102.3) (width 0.2) (layer "F.Cu") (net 8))
 (segment (start 153.224999 103.6) (end 153.9 103.6) (width 0.2) (layer "F.Cu") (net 7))
 (segment (start 153.9 103.6) (end 154.94 102.56) (width 0.2) (layer "F.Cu") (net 7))
 (segment (start 154.94 102.56) (end 154.94 99.06) (width 0.2) (layer "F.Cu") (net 7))
 (segment (start 151.375001 103.6) (end 151.375001 103.175001) (width 0.2) (layer "F.Cu") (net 1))
 (segment (start 149.86 101.66) (end 149.86 99.06) (width 0.2) (layer "F.Cu") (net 1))
 (segment (start 147.915 101.66) (end 147.775 101.8) (width 0.2) (layer "F.Cu") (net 1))
 (segment (start 151.375001 103.175001) (end 149.86 101.66) (width 0.2) (layer "F.Cu") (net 1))
 (segment (start 149.86 101.66) (end 147.915 101.66) (width 0.2) (layer "F.Cu") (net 1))
 (segment (start 152.405 107.005) (end 152.405 109.22) (width 0.2) (layer "F.Cu") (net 3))
 (segment (start 151.9 104.924999) (end 151.9 106.5) (width 0.2) (layer "F.Cu") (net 3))
 (segment (start 151.9 106.5) (end 152.405 107.005) (width 0.2) (layer "F.Cu") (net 3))
 (segment (start 153.5 107) (end 152.3 105.8) (width 0.2) (layer "F.Cu") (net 4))
 (segment (start 154.945 107.645) (end 154.3 107) (width 0.2) (layer "F.Cu") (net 4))
 (segment (start 154.3 107) (end 153.5 107) (width 0.2) (layer "F.Cu") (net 4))
 (segment (start 154.945 109.22) (end 154.945 107.645) (width 0.2) (layer "F.Cu") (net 4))
 (segment (start 152.3 105.8) (end 152.3 104.924999) (width 0.2) (layer "F.Cu") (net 4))
 (segment (start 153.224999 104) (end 154.3 104) (width 0.2) (layer "F.Cu") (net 2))
 (segment (start 146.35 103.65) (end 146.3 103.6) (width 0.2) (layer "F.Cu") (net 2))
 (segment (start 146.225 101.8) (end 146.225 103.525) (width 0.2) (layer "F.Cu") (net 2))
 (segment (start 146.225 103.525) (end 146.3 103.6) (width 0.2) (layer "F.Cu") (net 2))
 (segment (start 146.35 105.2) (end 146.35 103.65) (width 0.2) (layer "F.Cu") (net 2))
 (via (at 146.3 103.6) (size 0.8) (drill 0.4) (layers "F.Cu" "B.Cu") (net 2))
 (via (at 154.3 104) (size 0.8) (drill 0.4) (layers "F.Cu" "B.Cu") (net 2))
 (segment (start 151.375001 105.024999) (end 151.375001 104.4) (width 0.2) (layer "F.Cu") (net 12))
 (segment (start 147.9 105.2) (end 147.9 106.5) (width 0.2) (layer "F.Cu") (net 12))
 (segment (start 147.9 106.5) (end 149.9 106.5) (width 0.2) (layer "F.Cu") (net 12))
 (segment (start 147.325 107.075) (end 147.9 106.5) (width 0.2) (layer "F.Cu") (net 12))
 (segment (start 147.325 109.22) (end 147.325 107.075) (width 0.2) (layer "F.Cu") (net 12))
 (segment (start 149.9 106.5) (end 151.375001 105.024999) (width 0.2) (layer "F.Cu") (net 12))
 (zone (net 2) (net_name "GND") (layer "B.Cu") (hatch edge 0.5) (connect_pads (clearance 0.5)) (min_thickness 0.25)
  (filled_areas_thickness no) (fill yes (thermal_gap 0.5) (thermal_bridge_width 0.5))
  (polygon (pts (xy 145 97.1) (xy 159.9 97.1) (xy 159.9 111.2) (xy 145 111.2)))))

